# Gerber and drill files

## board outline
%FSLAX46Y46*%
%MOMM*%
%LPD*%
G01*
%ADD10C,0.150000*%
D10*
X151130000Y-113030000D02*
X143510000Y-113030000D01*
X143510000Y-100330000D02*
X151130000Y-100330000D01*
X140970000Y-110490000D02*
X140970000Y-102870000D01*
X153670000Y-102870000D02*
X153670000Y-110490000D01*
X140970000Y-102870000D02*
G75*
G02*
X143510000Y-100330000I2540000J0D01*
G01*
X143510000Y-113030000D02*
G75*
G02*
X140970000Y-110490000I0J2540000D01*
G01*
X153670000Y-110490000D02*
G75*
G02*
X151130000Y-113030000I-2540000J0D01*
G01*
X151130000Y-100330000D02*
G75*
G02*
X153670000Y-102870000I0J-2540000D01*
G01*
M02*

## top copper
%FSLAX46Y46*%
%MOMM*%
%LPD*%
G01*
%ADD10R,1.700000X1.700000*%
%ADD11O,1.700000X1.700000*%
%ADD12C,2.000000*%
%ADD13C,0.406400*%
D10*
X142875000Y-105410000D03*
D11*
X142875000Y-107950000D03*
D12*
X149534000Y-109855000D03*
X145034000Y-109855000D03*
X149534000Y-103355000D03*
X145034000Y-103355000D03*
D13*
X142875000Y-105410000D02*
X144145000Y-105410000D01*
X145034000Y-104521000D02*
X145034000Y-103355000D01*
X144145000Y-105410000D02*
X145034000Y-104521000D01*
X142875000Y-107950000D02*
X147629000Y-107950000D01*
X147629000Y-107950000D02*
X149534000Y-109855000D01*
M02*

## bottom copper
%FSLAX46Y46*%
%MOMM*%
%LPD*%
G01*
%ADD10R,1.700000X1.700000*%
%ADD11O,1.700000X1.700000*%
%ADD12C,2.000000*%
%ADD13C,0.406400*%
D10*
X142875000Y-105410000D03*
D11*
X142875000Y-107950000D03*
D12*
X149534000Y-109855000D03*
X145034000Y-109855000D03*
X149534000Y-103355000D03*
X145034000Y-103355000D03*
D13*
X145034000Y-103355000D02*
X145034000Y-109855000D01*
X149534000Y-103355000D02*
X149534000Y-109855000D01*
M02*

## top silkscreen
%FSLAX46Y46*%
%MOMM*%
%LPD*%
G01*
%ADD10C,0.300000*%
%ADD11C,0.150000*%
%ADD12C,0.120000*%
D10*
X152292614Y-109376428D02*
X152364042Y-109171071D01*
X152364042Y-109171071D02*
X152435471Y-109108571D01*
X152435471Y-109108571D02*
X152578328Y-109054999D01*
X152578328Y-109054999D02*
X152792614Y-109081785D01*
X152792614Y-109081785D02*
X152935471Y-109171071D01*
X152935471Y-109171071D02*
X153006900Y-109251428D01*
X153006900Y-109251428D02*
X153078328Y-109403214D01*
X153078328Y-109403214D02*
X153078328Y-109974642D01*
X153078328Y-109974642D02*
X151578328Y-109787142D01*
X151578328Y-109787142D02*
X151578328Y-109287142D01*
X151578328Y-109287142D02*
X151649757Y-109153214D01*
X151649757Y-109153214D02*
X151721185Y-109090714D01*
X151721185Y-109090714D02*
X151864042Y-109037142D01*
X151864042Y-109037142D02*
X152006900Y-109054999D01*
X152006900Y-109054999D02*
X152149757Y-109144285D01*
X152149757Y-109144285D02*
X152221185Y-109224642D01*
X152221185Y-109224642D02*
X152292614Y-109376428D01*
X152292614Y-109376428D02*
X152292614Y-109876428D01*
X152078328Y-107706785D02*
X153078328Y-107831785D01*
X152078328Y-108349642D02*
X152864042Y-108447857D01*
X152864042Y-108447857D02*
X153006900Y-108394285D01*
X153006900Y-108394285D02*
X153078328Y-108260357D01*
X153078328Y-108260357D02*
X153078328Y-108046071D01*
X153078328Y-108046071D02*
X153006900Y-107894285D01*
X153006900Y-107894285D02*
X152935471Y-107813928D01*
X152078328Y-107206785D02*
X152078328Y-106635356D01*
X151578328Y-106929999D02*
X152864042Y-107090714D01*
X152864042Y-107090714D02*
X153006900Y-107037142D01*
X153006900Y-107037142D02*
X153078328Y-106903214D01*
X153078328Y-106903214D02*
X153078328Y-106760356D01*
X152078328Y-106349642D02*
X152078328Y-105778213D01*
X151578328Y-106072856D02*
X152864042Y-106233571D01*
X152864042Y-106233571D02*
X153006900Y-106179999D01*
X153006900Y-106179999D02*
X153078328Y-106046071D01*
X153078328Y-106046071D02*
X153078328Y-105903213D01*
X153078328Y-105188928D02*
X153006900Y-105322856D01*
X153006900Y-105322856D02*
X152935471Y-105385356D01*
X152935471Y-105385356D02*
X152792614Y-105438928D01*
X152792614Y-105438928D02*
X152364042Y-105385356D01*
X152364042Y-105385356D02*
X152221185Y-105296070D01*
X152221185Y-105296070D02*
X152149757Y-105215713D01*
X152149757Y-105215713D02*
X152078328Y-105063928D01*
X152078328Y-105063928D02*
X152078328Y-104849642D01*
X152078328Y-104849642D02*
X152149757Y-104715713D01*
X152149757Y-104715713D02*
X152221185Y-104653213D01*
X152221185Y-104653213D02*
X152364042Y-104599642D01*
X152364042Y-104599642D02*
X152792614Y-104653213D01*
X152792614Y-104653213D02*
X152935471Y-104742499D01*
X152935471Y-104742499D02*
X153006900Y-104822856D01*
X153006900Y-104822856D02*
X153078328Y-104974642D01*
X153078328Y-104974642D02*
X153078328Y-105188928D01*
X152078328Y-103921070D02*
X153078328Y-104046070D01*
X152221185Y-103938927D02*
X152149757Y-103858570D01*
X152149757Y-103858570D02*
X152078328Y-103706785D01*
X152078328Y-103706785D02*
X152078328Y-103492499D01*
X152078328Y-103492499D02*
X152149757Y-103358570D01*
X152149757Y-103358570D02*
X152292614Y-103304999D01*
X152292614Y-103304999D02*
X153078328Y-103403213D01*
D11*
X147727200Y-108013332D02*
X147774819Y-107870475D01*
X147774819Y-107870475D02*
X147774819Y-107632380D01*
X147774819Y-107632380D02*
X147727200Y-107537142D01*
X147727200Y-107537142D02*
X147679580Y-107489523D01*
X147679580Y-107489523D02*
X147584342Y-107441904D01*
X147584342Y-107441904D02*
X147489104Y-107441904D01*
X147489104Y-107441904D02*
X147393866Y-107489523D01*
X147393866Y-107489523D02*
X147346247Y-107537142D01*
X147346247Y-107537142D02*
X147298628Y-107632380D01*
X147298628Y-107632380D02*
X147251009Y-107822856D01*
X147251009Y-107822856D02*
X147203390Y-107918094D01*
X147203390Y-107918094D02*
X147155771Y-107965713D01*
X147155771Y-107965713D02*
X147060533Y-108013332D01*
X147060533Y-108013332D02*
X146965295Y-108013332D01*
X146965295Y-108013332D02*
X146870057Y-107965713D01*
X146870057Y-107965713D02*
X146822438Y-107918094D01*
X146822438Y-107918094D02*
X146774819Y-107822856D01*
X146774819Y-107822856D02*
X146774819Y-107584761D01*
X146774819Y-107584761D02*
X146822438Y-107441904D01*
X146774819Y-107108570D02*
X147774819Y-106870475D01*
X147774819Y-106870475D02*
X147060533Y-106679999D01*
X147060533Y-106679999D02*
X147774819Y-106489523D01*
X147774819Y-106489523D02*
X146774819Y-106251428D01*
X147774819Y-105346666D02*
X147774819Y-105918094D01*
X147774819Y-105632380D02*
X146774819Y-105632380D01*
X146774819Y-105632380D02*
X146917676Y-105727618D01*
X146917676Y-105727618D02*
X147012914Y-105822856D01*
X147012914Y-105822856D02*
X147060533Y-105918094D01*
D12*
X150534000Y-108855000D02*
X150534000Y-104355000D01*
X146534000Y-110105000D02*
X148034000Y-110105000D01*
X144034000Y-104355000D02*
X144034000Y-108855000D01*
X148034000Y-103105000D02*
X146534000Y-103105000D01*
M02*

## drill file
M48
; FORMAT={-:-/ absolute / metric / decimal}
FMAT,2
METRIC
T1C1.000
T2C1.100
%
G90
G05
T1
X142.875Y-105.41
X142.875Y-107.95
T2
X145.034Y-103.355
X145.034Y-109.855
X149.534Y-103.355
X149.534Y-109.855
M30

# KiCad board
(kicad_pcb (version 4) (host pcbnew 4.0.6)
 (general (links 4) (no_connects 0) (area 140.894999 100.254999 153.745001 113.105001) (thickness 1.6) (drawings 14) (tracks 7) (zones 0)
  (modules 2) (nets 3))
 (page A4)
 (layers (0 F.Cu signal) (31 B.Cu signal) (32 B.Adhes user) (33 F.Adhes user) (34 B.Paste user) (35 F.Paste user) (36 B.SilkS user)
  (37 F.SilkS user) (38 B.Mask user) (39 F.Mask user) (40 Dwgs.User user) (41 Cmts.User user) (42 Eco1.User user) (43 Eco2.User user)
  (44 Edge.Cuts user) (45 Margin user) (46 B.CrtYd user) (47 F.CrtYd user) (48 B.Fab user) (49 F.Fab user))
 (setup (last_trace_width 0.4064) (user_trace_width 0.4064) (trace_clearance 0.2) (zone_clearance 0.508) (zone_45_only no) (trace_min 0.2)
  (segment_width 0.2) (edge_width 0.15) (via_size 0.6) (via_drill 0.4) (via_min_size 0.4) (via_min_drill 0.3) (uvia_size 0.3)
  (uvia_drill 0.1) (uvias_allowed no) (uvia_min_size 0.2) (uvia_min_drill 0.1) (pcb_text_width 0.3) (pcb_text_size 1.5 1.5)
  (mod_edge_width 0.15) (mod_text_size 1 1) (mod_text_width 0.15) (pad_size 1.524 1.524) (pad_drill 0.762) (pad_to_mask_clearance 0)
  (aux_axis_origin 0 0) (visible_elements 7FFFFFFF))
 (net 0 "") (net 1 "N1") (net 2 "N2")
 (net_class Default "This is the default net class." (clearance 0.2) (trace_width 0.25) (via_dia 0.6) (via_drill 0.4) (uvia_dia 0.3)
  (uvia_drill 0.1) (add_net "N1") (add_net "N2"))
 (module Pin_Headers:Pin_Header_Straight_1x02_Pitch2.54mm (layer F.Cu) (at 142.875 105.41)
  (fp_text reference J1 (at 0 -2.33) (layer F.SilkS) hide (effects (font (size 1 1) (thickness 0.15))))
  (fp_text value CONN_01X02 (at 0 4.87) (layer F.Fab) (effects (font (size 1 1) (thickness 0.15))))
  (pad 1 thru_hole rect (at 0 0) (size 1.7 1.7) (drill 1) (layers *.Cu *.Mask) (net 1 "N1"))
  (pad 2 thru_hole oval (at 0 2.54) (size 1.7 1.7) (drill 1) (layers *.Cu *.Mask) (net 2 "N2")))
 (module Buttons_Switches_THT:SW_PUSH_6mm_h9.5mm (layer F.Cu) (at 145.034 109.855 90)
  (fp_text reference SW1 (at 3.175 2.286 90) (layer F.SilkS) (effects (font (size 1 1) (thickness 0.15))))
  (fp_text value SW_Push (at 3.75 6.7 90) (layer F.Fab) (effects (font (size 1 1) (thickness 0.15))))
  (fp_line (start 1 5.5) (end 5.5 5.5) (layer F.SilkS) (width 0.12))
  (fp_line (start -0.25 1.5) (end -0.25 3) (layer F.SilkS) (width 0.12))
  (fp_line (start 5.5 -1) (end 1 -1) (layer F.SilkS) (width 0.12))
  (fp_line (start 6.75 3) (end 6.75 1.5) (layer F.SilkS) (width 0.12))
  (pad 2 thru_hole circle (at 0 4.5 180) (size 2 2) (drill 1.1) (layers *.Cu *.Mask) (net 2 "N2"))
  (pad 1 thru_hole circle (at 0 0 180) (size 2 2) (drill 1.1) (layers *.Cu *.Mask) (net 1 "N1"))
  (pad 2 thru_hole circle (at 6.5 4.5 180) (size 2 2) (drill 1.1) (layers *.Cu *.Mask) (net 2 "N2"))
  (pad 1 thru_hole circle (at 6.5 0 180) (size 2 2) (drill 1.1) (layers *.Cu *.Mask) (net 1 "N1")))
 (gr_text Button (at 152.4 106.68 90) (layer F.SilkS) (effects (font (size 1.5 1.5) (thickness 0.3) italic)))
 (gr_line (start 151.13 113.03) (end 143.51 113.03) (angle 90) (layer Edge.Cuts) (width 0.15))
 (gr_line (start 143.51 100.33) (end 151.13 100.33) (angle 90) (layer Edge.Cuts) (width 0.15))
 (gr_line (start 140.97 110.49) (end 140.97 102.87) (angle 90) (layer Edge.Cuts) (width 0.15))
 (gr_line (start 153.67 102.87) (end 153.67 110.49) (angle 90) (layer Edge.Cuts) (width 0.15))
 (gr_arc (start 143.51 102.87) (end 140.97 102.87) (angle 90) (layer Edge.Cuts) (width 0.15))
 (gr_arc (start 143.51 110.49) (end 143.51 113.03) (angle 90) (layer Edge.Cuts) (width 0.15))
 (gr_arc (start 151.13 110.49) (end 153.67 110.49) (angle 90) (layer Edge.Cuts) (width 0.15))
 (gr_arc (start 151.13 102.87) (end 151.13 100.33) (angle 90) (layer Edge.Cuts) (width 0.15))
 (segment (start 145.034 103.355) (end 145.034 109.855) (width 0.4064) (layer B.Cu) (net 1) (status C00000))
 (segment (start 142.875 105.41) (end 144.145 105.41) (width 0.4064) (layer F.Cu) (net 1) (status 400000))
 (segment (start 145.034 104.521) (end 145.034 103.355) (width 0.4064) (layer F.Cu) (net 1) (status 800000))
 (segment (start 144.145 105.41) (end 145.034 104.521) (width 0.4064) (layer F.Cu) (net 1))
 (segment (start 149.534 103.355) (end 149.534 109.855) (width 0.4064) (layer B.Cu) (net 2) (status C00000))
 (segment (start 142.875 107.95) (end 147.629 107.95) (width 0.4064) (layer F.Cu) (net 2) (status 400000))
 (segment (start 147.629 107.95) (end 149.534 109.855) (width 0.4064) (layer F.Cu) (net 2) (status 800000)))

